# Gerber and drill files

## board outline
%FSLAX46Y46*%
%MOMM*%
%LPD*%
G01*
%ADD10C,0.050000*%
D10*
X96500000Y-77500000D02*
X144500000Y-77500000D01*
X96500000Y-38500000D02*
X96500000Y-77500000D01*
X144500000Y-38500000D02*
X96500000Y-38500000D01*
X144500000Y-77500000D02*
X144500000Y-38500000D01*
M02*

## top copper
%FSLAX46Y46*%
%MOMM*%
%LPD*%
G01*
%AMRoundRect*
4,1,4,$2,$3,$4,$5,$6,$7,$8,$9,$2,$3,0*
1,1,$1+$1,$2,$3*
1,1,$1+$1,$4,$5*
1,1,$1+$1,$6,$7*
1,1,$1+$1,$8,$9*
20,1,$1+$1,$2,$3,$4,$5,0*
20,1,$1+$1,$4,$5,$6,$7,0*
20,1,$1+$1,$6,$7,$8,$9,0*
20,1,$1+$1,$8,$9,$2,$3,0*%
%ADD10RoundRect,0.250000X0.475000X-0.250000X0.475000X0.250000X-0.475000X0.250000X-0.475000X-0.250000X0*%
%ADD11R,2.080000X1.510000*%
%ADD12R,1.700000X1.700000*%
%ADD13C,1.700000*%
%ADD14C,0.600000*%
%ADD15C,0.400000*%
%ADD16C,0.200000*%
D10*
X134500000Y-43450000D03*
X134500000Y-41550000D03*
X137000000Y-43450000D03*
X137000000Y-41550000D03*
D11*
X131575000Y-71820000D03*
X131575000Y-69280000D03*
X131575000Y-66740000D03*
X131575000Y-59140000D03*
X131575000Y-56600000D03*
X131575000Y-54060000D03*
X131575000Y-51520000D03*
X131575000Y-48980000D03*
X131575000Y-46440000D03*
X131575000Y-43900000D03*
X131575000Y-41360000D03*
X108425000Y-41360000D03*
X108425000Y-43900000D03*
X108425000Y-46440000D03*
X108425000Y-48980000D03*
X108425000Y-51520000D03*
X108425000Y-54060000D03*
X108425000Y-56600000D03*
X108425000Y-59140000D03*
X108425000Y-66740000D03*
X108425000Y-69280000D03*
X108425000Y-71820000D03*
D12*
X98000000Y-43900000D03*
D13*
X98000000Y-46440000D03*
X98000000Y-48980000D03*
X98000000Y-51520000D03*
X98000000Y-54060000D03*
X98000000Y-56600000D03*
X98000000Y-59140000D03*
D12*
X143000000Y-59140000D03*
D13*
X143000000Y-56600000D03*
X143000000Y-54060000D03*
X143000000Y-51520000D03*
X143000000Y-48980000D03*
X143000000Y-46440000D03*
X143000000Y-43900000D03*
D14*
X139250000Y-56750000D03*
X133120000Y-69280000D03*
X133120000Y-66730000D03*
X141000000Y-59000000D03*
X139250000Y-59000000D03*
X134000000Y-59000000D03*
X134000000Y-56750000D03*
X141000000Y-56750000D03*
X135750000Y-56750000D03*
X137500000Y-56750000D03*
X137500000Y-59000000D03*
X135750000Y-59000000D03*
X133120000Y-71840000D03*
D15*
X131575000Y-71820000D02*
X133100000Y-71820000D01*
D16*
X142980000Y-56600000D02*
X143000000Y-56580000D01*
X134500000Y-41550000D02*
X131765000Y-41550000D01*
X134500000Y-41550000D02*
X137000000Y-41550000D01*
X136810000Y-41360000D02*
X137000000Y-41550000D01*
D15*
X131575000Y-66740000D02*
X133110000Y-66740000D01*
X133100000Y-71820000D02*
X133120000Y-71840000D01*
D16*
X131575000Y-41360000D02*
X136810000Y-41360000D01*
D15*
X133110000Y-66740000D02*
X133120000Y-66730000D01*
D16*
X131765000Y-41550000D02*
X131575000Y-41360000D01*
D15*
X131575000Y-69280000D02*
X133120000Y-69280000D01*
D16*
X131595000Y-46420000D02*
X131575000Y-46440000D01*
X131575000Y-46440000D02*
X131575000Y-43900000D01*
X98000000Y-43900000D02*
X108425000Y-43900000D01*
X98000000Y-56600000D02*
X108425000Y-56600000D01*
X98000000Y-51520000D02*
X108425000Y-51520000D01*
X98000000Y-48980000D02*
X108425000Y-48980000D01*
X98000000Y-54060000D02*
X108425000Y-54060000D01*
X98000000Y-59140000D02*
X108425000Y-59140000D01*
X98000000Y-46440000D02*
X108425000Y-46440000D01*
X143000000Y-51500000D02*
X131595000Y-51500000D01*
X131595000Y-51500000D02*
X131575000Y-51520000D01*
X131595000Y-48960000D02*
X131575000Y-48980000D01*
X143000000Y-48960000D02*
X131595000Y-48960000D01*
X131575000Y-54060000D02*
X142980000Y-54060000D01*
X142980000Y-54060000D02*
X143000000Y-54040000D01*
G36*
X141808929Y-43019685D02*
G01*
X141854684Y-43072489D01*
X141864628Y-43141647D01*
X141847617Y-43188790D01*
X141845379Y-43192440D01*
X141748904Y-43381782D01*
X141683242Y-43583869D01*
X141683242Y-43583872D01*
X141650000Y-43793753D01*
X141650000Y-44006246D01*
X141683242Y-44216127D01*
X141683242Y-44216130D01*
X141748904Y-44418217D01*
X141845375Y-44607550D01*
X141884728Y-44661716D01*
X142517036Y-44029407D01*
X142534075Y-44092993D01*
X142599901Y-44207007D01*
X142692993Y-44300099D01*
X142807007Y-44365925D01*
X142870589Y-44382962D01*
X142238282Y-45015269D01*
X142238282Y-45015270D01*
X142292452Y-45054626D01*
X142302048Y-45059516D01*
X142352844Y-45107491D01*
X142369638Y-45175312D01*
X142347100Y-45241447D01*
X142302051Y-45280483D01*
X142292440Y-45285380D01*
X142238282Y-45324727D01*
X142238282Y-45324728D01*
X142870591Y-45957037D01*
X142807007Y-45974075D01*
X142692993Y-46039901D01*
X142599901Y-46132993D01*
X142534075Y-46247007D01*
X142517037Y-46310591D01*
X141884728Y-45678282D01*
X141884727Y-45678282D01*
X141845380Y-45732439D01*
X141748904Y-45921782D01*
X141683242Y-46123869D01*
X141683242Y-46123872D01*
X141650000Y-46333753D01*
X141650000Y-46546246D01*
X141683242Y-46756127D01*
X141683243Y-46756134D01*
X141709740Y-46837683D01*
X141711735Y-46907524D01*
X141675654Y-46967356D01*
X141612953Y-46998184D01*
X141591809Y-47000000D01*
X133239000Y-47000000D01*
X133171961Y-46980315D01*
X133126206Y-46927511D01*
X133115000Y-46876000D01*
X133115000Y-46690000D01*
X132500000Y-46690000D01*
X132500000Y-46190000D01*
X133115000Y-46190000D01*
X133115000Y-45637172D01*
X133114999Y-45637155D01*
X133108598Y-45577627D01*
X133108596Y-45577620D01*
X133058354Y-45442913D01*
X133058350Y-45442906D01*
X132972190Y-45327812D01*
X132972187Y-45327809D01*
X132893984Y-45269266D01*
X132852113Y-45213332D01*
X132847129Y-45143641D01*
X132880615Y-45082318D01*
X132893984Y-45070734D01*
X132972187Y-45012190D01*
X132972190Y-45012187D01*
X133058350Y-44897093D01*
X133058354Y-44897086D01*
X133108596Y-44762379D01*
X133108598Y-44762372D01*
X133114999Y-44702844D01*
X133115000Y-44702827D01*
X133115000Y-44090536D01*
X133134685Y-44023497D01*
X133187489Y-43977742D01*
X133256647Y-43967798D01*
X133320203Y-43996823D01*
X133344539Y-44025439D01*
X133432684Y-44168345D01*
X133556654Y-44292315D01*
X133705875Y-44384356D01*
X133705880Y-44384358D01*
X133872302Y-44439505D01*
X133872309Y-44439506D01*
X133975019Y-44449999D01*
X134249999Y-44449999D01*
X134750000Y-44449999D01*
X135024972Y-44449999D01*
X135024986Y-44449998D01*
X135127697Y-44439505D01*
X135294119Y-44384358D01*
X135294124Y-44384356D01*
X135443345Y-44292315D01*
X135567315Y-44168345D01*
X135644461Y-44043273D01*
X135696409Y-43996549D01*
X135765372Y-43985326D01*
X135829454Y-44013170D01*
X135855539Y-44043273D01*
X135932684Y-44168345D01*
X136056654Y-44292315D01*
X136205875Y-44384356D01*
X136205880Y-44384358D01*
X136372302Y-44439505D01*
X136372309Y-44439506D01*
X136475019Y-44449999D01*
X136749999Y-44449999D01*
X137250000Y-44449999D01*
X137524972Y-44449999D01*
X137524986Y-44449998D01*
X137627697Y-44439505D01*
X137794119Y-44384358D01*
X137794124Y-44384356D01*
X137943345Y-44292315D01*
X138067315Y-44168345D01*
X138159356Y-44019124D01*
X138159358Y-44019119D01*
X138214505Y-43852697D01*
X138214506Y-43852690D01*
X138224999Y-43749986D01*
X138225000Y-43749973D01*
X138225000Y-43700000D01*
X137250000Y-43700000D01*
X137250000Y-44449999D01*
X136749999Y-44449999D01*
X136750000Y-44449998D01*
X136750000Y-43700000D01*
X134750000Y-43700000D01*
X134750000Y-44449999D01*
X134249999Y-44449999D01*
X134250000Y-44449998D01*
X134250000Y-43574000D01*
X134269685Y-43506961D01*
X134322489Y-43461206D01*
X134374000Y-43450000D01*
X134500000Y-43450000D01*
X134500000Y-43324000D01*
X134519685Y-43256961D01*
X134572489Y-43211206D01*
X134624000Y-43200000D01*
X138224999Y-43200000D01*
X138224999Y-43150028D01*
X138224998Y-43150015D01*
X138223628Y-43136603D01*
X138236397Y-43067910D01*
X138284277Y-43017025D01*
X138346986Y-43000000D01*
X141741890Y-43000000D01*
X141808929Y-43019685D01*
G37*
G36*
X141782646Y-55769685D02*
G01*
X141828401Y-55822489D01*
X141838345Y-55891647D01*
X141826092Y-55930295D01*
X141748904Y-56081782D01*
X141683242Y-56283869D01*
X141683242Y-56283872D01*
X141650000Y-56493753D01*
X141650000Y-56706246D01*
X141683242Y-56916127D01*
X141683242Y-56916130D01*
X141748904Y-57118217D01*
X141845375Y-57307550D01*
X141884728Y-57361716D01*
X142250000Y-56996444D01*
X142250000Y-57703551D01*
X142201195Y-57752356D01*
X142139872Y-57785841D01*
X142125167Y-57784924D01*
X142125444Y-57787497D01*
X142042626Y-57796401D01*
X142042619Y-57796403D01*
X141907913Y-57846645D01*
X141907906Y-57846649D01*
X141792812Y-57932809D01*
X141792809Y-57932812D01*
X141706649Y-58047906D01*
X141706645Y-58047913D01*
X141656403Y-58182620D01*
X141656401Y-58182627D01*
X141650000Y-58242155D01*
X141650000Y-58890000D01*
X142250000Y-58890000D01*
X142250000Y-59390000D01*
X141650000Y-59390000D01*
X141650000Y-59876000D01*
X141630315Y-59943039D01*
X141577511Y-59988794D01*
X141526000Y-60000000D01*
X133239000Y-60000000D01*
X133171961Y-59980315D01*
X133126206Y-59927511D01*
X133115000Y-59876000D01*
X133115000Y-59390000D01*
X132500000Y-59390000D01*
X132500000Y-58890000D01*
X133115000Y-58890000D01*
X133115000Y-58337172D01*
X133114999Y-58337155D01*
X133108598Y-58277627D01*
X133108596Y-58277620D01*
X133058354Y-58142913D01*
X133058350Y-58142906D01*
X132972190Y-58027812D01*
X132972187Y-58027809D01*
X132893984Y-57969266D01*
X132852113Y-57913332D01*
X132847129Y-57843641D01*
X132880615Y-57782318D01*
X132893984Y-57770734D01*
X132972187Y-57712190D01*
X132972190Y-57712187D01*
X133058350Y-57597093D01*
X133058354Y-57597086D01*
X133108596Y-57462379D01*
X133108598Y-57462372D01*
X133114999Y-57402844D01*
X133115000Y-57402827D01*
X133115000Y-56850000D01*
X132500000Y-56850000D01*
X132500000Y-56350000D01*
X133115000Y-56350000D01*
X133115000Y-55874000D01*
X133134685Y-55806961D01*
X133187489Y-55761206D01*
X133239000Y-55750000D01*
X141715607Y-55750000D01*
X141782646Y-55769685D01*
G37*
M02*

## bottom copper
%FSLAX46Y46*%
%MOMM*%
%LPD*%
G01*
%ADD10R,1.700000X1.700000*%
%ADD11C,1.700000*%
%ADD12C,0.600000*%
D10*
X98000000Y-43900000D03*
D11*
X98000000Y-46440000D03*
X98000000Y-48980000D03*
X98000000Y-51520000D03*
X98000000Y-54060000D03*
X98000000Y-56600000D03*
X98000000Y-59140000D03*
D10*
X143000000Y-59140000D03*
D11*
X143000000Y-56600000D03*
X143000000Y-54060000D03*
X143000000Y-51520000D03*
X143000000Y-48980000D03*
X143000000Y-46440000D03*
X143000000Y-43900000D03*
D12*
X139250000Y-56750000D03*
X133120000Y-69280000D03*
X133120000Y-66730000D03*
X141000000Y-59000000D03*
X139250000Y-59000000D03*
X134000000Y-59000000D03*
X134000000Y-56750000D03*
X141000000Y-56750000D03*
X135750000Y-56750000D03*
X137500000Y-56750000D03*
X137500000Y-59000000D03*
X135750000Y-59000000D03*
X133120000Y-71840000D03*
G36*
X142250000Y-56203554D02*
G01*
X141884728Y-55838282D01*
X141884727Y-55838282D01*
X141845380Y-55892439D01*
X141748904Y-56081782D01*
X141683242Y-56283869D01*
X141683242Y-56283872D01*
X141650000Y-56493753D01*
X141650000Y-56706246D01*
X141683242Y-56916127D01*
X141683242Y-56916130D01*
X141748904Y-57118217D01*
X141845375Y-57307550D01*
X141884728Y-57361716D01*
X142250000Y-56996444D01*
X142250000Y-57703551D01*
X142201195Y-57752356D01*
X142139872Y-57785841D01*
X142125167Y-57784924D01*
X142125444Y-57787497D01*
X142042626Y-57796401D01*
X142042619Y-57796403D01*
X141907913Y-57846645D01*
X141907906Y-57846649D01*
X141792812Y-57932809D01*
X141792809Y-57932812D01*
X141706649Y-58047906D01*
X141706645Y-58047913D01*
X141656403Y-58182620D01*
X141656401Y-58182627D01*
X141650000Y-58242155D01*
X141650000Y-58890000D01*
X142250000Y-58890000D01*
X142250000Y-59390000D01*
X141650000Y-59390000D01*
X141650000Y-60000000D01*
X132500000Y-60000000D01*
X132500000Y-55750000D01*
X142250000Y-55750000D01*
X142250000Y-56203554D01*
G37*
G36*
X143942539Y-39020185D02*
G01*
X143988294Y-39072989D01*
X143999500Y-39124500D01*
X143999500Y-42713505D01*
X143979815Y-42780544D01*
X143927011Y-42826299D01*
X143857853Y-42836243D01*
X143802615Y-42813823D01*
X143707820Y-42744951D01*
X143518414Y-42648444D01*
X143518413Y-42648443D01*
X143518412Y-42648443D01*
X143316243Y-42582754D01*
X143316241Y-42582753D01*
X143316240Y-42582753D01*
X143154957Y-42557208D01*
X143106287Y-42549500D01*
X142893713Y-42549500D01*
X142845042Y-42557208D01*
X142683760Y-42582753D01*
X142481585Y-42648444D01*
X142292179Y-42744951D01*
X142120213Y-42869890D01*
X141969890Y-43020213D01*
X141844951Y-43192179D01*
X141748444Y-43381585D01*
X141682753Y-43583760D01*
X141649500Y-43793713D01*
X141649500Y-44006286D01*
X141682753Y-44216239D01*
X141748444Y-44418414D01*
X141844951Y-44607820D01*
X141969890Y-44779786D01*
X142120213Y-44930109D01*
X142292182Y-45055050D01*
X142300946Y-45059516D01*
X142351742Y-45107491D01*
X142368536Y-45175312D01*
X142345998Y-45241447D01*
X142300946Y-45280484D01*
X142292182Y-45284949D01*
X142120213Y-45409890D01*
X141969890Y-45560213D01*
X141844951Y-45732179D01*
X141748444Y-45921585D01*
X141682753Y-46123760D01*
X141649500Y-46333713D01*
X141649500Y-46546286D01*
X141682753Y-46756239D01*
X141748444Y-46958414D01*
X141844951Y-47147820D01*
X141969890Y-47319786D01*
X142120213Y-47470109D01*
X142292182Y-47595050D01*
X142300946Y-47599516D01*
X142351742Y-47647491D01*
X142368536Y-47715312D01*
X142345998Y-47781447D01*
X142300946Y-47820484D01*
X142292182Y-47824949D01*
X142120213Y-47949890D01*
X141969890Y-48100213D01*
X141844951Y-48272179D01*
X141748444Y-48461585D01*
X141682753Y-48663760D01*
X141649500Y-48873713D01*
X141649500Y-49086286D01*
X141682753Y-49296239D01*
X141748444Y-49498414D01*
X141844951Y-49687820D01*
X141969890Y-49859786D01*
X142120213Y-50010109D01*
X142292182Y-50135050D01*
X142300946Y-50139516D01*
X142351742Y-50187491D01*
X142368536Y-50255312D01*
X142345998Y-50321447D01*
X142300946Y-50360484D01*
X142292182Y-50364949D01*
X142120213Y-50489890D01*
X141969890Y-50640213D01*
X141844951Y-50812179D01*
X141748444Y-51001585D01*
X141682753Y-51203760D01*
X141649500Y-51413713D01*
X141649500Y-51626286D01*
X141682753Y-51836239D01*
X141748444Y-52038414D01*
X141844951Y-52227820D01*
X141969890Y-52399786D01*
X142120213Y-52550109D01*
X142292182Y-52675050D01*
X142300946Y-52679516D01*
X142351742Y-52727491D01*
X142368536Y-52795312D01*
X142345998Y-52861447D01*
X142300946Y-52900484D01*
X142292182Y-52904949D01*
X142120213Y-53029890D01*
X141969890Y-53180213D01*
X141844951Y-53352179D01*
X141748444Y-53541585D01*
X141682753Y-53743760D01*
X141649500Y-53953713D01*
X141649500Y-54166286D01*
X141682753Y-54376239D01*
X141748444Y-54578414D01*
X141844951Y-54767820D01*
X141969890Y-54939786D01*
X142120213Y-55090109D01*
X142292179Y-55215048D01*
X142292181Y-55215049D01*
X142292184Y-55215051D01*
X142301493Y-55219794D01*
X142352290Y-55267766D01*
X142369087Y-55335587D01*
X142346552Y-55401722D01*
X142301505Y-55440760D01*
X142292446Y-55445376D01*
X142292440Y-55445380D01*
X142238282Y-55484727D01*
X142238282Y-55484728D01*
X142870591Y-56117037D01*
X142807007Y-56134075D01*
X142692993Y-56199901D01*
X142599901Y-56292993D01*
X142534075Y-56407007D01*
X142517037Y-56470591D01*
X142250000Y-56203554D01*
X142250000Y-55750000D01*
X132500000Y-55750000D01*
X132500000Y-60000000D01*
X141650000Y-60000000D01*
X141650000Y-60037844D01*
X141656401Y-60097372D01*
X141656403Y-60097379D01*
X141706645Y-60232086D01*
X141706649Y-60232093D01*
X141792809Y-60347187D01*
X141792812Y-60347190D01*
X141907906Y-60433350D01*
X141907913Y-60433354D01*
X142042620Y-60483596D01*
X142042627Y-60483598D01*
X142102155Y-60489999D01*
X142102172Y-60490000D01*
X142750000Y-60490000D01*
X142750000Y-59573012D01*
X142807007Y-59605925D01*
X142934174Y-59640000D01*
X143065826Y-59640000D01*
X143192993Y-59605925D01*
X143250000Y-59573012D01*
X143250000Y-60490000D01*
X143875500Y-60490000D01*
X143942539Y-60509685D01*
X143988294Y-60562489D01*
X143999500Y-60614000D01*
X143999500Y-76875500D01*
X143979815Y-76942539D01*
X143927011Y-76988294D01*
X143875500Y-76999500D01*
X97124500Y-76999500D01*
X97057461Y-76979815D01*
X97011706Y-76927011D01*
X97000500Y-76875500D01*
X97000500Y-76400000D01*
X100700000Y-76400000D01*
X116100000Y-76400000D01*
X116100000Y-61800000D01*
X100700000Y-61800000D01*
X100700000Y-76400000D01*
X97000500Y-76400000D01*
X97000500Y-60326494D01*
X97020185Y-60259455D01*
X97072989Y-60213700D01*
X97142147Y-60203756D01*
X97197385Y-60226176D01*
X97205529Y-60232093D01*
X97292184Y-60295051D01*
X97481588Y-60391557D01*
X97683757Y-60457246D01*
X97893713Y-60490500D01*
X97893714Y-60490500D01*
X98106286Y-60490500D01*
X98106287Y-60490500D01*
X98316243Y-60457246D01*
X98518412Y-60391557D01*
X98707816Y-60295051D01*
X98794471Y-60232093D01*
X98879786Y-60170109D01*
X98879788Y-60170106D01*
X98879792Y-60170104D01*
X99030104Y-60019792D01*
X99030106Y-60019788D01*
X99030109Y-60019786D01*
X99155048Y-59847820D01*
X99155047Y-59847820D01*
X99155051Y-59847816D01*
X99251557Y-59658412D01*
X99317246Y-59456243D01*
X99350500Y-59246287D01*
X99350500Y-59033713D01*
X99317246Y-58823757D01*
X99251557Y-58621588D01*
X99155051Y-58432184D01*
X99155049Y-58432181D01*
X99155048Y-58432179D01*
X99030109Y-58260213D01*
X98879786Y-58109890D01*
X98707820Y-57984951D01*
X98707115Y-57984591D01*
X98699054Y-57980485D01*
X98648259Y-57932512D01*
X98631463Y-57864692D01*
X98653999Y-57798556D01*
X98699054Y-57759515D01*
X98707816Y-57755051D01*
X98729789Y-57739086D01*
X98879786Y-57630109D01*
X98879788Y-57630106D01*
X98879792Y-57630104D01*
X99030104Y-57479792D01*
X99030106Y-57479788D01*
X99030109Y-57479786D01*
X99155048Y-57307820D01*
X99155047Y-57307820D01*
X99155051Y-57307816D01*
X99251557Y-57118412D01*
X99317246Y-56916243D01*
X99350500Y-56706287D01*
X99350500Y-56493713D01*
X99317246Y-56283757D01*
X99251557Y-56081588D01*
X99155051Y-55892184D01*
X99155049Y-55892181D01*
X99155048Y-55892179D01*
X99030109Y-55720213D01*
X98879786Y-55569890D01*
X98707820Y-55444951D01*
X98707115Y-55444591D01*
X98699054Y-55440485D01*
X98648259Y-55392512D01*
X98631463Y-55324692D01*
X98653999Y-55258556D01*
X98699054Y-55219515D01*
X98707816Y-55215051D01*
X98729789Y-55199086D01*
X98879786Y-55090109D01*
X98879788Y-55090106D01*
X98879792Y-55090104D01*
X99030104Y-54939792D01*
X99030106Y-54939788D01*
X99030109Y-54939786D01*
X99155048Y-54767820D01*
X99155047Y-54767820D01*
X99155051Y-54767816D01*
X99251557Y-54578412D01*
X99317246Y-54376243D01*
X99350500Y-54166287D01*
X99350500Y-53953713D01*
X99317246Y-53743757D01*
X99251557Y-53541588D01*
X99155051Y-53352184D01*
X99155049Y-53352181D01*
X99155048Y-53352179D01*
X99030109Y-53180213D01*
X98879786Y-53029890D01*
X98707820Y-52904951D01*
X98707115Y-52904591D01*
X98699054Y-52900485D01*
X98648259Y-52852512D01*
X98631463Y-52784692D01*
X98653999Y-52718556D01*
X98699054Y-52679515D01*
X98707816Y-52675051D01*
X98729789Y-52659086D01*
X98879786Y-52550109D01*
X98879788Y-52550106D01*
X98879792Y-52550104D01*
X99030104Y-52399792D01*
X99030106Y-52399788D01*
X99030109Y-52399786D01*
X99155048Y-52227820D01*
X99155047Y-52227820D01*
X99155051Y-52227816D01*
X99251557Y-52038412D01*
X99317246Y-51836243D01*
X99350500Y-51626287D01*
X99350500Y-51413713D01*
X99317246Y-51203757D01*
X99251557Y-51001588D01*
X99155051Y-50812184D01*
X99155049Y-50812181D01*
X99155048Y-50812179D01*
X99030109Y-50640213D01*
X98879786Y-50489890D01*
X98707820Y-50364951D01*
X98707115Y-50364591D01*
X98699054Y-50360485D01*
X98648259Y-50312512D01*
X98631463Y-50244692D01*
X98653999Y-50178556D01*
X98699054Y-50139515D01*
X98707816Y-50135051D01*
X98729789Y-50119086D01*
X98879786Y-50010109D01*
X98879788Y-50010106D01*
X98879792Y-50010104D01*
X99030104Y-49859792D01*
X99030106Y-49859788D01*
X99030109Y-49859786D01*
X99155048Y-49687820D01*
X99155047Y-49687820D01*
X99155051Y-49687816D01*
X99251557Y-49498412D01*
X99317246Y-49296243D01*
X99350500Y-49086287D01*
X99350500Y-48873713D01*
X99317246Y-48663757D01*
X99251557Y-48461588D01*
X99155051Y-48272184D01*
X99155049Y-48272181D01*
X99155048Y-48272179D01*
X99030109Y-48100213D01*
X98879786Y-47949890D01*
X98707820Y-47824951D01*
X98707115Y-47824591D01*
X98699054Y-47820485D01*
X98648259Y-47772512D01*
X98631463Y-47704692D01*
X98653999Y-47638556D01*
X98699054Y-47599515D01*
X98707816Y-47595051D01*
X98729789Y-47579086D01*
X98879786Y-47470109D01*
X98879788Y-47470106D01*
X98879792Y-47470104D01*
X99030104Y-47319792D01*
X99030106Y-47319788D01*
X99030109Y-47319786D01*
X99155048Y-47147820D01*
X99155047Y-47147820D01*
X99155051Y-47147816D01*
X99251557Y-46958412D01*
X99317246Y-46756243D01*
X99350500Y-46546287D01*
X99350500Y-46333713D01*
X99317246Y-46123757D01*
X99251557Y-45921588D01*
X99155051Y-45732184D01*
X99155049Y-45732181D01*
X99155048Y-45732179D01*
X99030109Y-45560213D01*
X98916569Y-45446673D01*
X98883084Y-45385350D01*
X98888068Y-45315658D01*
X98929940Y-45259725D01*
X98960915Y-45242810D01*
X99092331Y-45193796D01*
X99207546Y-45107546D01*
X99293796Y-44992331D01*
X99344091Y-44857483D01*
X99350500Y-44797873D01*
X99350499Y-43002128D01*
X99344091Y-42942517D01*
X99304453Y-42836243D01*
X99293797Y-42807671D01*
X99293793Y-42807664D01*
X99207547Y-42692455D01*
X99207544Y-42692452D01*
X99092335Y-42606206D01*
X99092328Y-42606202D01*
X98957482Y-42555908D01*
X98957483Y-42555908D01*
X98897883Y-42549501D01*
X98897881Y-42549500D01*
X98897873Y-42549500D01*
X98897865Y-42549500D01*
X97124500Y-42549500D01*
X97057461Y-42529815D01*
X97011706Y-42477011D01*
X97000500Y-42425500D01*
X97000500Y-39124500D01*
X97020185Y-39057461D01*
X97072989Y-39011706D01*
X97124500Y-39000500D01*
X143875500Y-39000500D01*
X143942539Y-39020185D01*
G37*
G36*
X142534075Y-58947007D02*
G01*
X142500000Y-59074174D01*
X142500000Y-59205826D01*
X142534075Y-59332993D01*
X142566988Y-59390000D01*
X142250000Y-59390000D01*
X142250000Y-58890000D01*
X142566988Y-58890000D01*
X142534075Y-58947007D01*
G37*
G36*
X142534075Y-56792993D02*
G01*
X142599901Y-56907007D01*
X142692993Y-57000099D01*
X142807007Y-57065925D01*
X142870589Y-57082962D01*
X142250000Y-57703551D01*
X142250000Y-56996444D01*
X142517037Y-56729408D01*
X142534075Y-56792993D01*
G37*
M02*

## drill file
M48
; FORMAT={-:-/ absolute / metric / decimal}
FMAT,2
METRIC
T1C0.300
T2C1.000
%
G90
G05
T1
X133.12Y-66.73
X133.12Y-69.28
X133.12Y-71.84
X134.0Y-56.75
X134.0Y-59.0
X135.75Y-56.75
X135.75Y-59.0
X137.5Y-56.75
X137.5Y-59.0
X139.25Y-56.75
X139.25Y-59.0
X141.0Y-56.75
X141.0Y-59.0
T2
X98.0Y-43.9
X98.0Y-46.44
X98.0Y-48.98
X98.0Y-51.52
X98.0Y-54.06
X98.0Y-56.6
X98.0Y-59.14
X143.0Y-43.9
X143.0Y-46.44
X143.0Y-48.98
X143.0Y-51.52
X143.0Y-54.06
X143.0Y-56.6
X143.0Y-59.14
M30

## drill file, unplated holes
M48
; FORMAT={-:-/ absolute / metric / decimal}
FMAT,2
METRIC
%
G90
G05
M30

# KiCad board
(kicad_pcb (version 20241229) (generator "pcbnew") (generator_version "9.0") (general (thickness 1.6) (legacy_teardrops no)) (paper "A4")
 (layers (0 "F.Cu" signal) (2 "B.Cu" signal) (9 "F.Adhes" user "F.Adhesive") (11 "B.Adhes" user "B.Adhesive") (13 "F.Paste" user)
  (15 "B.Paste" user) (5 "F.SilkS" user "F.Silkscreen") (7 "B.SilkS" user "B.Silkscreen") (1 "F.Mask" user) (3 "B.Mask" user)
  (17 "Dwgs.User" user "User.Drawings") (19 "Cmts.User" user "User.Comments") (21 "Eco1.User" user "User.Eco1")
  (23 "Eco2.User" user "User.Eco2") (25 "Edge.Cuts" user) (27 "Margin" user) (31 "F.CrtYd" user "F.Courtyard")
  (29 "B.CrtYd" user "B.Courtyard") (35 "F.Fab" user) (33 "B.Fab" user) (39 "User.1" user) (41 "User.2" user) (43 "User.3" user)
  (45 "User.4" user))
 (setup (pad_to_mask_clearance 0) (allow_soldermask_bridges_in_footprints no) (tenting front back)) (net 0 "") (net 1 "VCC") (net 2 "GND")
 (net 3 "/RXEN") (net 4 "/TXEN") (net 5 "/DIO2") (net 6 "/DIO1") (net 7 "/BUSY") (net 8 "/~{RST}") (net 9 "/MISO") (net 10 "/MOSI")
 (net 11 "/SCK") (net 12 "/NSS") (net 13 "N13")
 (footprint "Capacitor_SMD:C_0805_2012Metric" (layer "F.Cu") (at 134.5 42.5 90)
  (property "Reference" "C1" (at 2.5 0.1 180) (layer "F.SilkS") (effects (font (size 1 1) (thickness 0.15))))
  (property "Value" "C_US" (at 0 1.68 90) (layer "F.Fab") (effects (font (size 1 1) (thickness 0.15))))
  (pad "1" smd roundrect (at -0.95 0 90) (size 1 1.45) (layers "F.Cu" "F.Mask" "F.Paste") (roundrect_rratio 0.25) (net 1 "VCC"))
  (pad "2" smd roundrect (at 0.95 0 90) (size 1 1.45) (layers "F.Cu" "F.Mask" "F.Paste") (roundrect_rratio 0.25) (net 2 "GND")))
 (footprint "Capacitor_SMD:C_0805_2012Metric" (layer "F.Cu") (at 137 42.5 90)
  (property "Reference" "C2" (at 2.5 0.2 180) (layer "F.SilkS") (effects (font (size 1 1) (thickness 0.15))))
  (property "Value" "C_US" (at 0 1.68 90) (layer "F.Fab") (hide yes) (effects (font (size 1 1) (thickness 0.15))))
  (pad "1" smd roundrect (at -0.95 0 90) (size 1 1.45) (layers "F.Cu" "F.Mask" "F.Paste") (roundrect_rratio 0.25) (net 1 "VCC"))
  (pad "2" smd roundrect (at 0.95 0 90) (size 1 1.45) (layers "F.Cu" "F.Mask" "F.Paste") (roundrect_rratio 0.25) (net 2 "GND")))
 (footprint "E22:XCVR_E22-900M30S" (layer "F.Cu") (at 120 58)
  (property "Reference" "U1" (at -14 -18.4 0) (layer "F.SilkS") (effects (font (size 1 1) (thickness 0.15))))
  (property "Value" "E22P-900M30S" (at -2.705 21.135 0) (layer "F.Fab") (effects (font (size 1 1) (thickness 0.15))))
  (pad "1" smd rect (at 11.575 13.82) (size 2.08 1.51) (layers "F.Cu" "F.Mask" "F.Paste") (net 2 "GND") (solder_mask_margin 0.102))
  (pad "2" smd rect (at 11.575 11.28) (size 2.08 1.51) (layers "F.Cu" "F.Mask" "F.Paste") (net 2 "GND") (solder_mask_margin 0.102))
  (pad "3" smd rect (at 11.575 8.74) (size 2.08 1.51) (layers "F.Cu" "F.Mask" "F.Paste") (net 2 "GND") (solder_mask_margin 0.102))
  (pad "4" smd rect (at 11.575 1.14) (size 2.08 1.51) (layers "F.Cu" "F.Mask" "F.Paste") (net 2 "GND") (solder_mask_margin 0.102))
  (pad "5" smd rect (at 11.575 -1.4) (size 2.08 1.51) (layers "F.Cu" "F.Mask" "F.Paste") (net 2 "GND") (solder_mask_margin 0.102))
  (pad "6" smd rect (at 11.575 -3.94) (size 2.08 1.51) (layers "F.Cu" "F.Mask" "F.Paste") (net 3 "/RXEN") (solder_mask_margin 0.102))
  (pad "7" smd rect (at 11.575 -6.48) (size 2.08 1.51) (layers "F.Cu" "F.Mask" "F.Paste") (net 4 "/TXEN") (solder_mask_margin 0.102))
  (pad "8" smd rect (at 11.575 -9.02) (size 2.08 1.51) (layers "F.Cu" "F.Mask" "F.Paste") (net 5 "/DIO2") (solder_mask_margin 0.102))
  (pad "9" smd rect (at 11.575 -11.56) (size 2.08 1.51) (layers "F.Cu" "F.Mask" "F.Paste") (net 1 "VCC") (solder_mask_margin 0.102))
  (pad "10" smd rect (at 11.575 -14.1) (size 2.08 1.51) (layers "F.Cu" "F.Mask" "F.Paste") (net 1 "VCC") (solder_mask_margin 0.102))
  (pad "11" smd rect (at 11.575 -16.64) (size 2.08 1.51) (layers "F.Cu" "F.Mask" "F.Paste") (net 2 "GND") (solder_mask_margin 0.102))
  (pad "12" smd rect (at -11.575 -16.64) (size 2.08 1.51) (layers "F.Cu" "F.Mask" "F.Paste") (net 2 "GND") (solder_mask_margin 0.102))
  (pad "13" smd rect (at -11.575 -14.1) (size 2.08 1.51) (layers "F.Cu" "F.Mask" "F.Paste") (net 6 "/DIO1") (solder_mask_margin 0.102))
  (pad "14" smd rect (at -11.575 -11.56) (size 2.08 1.51) (layers "F.Cu" "F.Mask" "F.Paste") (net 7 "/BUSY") (solder_mask_margin 0.102))
  (pad "15" smd rect (at -11.575 -9.02) (size 2.08 1.51) (layers "F.Cu" "F.Mask" "F.Paste") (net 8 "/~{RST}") (solder_mask_margin 0.102))
  (pad "16" smd rect (at -11.575 -6.48) (size 2.08 1.51) (layers "F.Cu" "F.Mask" "F.Paste") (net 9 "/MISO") (solder_mask_margin 0.102))
  (pad "17" smd rect (at -11.575 -3.94) (size 2.08 1.51) (layers "F.Cu" "F.Mask" "F.Paste") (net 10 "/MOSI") (solder_mask_margin 0.102))
  (pad "18" smd rect (at -11.575 -1.4) (size 2.08 1.51) (layers "F.Cu" "F.Mask" "F.Paste") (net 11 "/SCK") (solder_mask_margin 0.102))
  (pad "19" smd rect (at -11.575 1.14) (size 2.08 1.51) (layers "F.Cu" "F.Mask" "F.Paste") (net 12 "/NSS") (solder_mask_margin 0.102))
  (pad "20" smd rect (at -11.575 8.74) (size 2.08 1.51) (layers "F.Cu" "F.Mask" "F.Paste") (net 2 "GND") (solder_mask_margin 0.102))
  (pad "21" smd rect (at -11.575 11.28) (size 2.08 1.51) (layers "F.Cu" "F.Mask" "F.Paste") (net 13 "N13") (solder_mask_margin 0.102))
  (pad "22" smd rect (at -11.575 13.82) (size 2.08 1.51) (layers "F.Cu" "F.Mask" "F.Paste") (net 2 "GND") (solder_mask_margin 0.102)))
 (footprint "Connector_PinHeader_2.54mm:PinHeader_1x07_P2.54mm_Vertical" (layer "B.Cu") (at 98 43.9 180)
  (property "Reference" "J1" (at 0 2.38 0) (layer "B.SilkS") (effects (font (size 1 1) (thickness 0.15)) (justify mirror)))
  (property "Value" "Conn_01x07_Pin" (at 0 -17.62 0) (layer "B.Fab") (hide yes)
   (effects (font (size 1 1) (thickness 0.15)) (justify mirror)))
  (pad "1" thru_hole rect (at 0 0 180) (size 1.7 1.7) (drill 1) (layers "*.Cu" "*.Mask") (remove_unused_layers no) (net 6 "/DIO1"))
  (pad "2" thru_hole circle (at 0 -2.54 180) (size 1.7 1.7) (drill 1) (layers "*.Cu" "*.Mask") (remove_unused_layers no) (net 7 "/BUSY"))
  (pad "3" thru_hole circle (at 0 -5.08 180) (size 1.7 1.7) (drill 1) (layers "*.Cu" "*.Mask") (remove_unused_layers no) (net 8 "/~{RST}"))
  (pad "4" thru_hole circle (at 0 -7.62 180) (size 1.7 1.7) (drill 1) (layers "*.Cu" "*.Mask") (remove_unused_layers no) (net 9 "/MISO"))
  (pad "5" thru_hole circle (at 0 -10.16 180) (size 1.7 1.7) (drill 1) (layers "*.Cu" "*.Mask") (remove_unused_layers no) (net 10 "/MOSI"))
  (pad "6" thru_hole circle (at 0 -12.7 180) (size 1.7 1.7) (drill 1) (layers "*.Cu" "*.Mask") (remove_unused_layers no) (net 11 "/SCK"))
  (pad "7" thru_hole circle (at 0 -15.24 180) (size 1.7 1.7) (drill 1) (layers "*.Cu" "*.Mask") (remove_unused_layers no) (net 12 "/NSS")))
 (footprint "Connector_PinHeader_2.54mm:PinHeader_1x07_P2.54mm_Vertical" (layer "B.Cu") (at 143 59.14)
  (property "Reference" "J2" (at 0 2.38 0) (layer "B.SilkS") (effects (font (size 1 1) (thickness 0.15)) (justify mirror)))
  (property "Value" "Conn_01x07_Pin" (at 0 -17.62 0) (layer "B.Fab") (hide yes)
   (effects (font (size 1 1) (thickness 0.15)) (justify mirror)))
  (pad "1" thru_hole rect (at 0 0) (size 1.7 1.7) (drill 1) (layers "*.Cu" "*.Mask") (remove_unused_layers no) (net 2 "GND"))
  (pad "2" thru_hole circle (at 0 -2.54) (size 1.7 1.7) (drill 1) (layers "*.Cu" "*.Mask") (remove_unused_layers no) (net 2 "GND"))
  (pad "3" thru_hole circle (at 0 -5.08) (size 1.7 1.7) (drill 1) (layers "*.Cu" "*.Mask") (remove_unused_layers no) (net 3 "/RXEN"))
  (pad "4" thru_hole circle (at 0 -7.62) (size 1.7 1.7) (drill 1) (layers "*.Cu" "*.Mask") (remove_unused_layers no) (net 4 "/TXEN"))
  (pad "5" thru_hole circle (at 0 -10.16) (size 1.7 1.7) (drill 1) (layers "*.Cu" "*.Mask") (remove_unused_layers no) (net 5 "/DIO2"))
  (pad "6" thru_hole circle (at 0 -12.7) (size 1.7 1.7) (drill 1) (layers "*.Cu" "*.Mask") (remove_unused_layers no) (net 1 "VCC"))
  (pad "7" thru_hole circle (at 0 -15.24) (size 1.7 1.7) (drill 1) (layers "*.Cu" "*.Mask") (remove_unused_layers no) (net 1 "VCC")))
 (gr_line (start 96.5 77.5) (end 144.5 77.5) (stroke (width 0.05) (type default)) (layer "Edge.Cuts"))
 (gr_line (start 96.5 38.5) (end 96.5 77.5) (stroke (width 0.05) (type default)) (layer "Edge.Cuts"))
 (gr_line (start 144.5 38.5) (end 96.5 38.5) (stroke (width 0.05) (type default)) (layer "Edge.Cuts"))
 (gr_line (start 144.5 77.5) (end 144.5 38.5) (stroke (width 0.05) (type default)) (layer "Edge.Cuts"))
 (segment (start 131.575 71.82) (end 133.1 71.82) (width 0.4) (layer "F.Cu") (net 2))
 (segment (start 142.98 56.6) (end 143 56.58) (width 0.2) (layer "F.Cu") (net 2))
 (segment (start 134.5 41.55) (end 131.765 41.55) (width 0.2) (layer "F.Cu") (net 2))
 (segment (start 134.5 41.55) (end 137 41.55) (width 0.2) (layer "F.Cu") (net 2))
 (segment (start 136.81 41.36) (end 137 41.55) (width 0.2) (layer "F.Cu") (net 2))
 (segment (start 131.575 66.74) (end 133.11 66.74) (width 0.4) (layer "F.Cu") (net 2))
 (segment (start 133.1 71.82) (end 133.12 71.84) (width 0.4) (layer "F.Cu") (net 2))
 (segment (start 131.575 41.36) (end 136.81 41.36) (width 0.2) (layer "F.Cu") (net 2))
 (segment (start 133.11 66.74) (end 133.12 66.73) (width 0.4) (layer "F.Cu") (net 2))
 (segment (start 131.765 41.55) (end 131.575 41.36) (width 0.2) (layer "F.Cu") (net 2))
 (segment (start 131.575 69.28) (end 133.12 69.28) (width 0.4) (layer "F.Cu") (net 2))
 (via (at 139.25 56.75) (size 0.6) (drill 0.3) (layers "F.Cu" "B.Cu") (free yes) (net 2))
 (via (at 133.12 69.28) (size 0.6) (drill 0.3) (layers "F.Cu" "B.Cu") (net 2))
 (via (at 133.12 66.73) (size 0.6) (drill 0.3) (layers "F.Cu" "B.Cu") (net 2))
 (via (at 141 59) (size 0.6) (drill 0.3) (layers "F.Cu" "B.Cu") (free yes) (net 2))
 (via (at 139.25 59) (size 0.6) (drill 0.3) (layers "F.Cu" "B.Cu") (free yes) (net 2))
 (via (at 134 59) (size 0.6) (drill 0.3) (layers "F.Cu" "B.Cu") (free yes) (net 2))
 (via (at 134 56.75) (size 0.6) (drill 0.3) (layers "F.Cu" "B.Cu") (free yes) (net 2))
 (via (at 141 56.75) (size 0.6) (drill 0.3) (layers "F.Cu" "B.Cu") (free yes) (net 2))
 (via (at 135.75 56.75) (size 0.6) (drill 0.3) (layers "F.Cu" "B.Cu") (free yes) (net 2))
 (via (at 137.5 56.75) (size 0.6) (drill 0.3) (layers "F.Cu" "B.Cu") (free yes) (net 2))
 (via (at 137.5 59) (size 0.6) (drill 0.3) (layers "F.Cu" "B.Cu") (free yes) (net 2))
 (via (at 135.75 59) (size 0.6) (drill 0.3) (layers "F.Cu" "B.Cu") (free yes) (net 2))
 (via (at 133.12 71.84) (size 0.6) (drill 0.3) (layers "F.Cu" "B.Cu") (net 2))
 (segment (start 131.595 46.42) (end 131.575 46.44) (width 0.2) (layer "F.Cu") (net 1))
 (segment (start 131.575 46.44) (end 131.575 43.9) (width 0.2) (layer "F.Cu") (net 1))
 (segment (start 98 43.9) (end 108.425 43.9) (width 0.2) (layer "F.Cu") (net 6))
 (segment (start 98 56.6) (end 108.425 56.6) (width 0.2) (layer "F.Cu") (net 11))
 (segment (start 98 51.52) (end 108.425 51.52) (width 0.2) (layer "F.Cu") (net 9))
 (segment (start 98 48.98) (end 108.425 48.98) (width 0.2) (layer "F.Cu") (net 8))
 (segment (start 98 54.06) (end 108.425 54.06) (width 0.2) (layer "F.Cu") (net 10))
 (segment (start 98 59.14) (end 108.425 59.14) (width 0.2) (layer "F.Cu") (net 12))
 (segment (start 98 46.44) (end 108.425 46.44) (width 0.2) (layer "F.Cu") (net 7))
 (segment (start 143 51.5) (end 131.595 51.5) (width 0.2) (layer "F.Cu") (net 4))
 (segment (start 131.595 51.5) (end 131.575 51.52) (width 0.2) (layer "F.Cu") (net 4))
 (segment (start 131.595 48.96) (end 131.575 48.98) (width 0.2) (layer "F.Cu") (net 5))
 (segment (start 143 48.96) (end 131.595 48.96) (width 0.2) (layer "F.Cu") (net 5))
 (segment (start 131.575 54.06) (end 142.98 54.06) (width 0.2) (layer "F.Cu") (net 3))
 (segment (start 142.98 54.06) (end 143 54.04) (width 0.2) (layer "F.Cu") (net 3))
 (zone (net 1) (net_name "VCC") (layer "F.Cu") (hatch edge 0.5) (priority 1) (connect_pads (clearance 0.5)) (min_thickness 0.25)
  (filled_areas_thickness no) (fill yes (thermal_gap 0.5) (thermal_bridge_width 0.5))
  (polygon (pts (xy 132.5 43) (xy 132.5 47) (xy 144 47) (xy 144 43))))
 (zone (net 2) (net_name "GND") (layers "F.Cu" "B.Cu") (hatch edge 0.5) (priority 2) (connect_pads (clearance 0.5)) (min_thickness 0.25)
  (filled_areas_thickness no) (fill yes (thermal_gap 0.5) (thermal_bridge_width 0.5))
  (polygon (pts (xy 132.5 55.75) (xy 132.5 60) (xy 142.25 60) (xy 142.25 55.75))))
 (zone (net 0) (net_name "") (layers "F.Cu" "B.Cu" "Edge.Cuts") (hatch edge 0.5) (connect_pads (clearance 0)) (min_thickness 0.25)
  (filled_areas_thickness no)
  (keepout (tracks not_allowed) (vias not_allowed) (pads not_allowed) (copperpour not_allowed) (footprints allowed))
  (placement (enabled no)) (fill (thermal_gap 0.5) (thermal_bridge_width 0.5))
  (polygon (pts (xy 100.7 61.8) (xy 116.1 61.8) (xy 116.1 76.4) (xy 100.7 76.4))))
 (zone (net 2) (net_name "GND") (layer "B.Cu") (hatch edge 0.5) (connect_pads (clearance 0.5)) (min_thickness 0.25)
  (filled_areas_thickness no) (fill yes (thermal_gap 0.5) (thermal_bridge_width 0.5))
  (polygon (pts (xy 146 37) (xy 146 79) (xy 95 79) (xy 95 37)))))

